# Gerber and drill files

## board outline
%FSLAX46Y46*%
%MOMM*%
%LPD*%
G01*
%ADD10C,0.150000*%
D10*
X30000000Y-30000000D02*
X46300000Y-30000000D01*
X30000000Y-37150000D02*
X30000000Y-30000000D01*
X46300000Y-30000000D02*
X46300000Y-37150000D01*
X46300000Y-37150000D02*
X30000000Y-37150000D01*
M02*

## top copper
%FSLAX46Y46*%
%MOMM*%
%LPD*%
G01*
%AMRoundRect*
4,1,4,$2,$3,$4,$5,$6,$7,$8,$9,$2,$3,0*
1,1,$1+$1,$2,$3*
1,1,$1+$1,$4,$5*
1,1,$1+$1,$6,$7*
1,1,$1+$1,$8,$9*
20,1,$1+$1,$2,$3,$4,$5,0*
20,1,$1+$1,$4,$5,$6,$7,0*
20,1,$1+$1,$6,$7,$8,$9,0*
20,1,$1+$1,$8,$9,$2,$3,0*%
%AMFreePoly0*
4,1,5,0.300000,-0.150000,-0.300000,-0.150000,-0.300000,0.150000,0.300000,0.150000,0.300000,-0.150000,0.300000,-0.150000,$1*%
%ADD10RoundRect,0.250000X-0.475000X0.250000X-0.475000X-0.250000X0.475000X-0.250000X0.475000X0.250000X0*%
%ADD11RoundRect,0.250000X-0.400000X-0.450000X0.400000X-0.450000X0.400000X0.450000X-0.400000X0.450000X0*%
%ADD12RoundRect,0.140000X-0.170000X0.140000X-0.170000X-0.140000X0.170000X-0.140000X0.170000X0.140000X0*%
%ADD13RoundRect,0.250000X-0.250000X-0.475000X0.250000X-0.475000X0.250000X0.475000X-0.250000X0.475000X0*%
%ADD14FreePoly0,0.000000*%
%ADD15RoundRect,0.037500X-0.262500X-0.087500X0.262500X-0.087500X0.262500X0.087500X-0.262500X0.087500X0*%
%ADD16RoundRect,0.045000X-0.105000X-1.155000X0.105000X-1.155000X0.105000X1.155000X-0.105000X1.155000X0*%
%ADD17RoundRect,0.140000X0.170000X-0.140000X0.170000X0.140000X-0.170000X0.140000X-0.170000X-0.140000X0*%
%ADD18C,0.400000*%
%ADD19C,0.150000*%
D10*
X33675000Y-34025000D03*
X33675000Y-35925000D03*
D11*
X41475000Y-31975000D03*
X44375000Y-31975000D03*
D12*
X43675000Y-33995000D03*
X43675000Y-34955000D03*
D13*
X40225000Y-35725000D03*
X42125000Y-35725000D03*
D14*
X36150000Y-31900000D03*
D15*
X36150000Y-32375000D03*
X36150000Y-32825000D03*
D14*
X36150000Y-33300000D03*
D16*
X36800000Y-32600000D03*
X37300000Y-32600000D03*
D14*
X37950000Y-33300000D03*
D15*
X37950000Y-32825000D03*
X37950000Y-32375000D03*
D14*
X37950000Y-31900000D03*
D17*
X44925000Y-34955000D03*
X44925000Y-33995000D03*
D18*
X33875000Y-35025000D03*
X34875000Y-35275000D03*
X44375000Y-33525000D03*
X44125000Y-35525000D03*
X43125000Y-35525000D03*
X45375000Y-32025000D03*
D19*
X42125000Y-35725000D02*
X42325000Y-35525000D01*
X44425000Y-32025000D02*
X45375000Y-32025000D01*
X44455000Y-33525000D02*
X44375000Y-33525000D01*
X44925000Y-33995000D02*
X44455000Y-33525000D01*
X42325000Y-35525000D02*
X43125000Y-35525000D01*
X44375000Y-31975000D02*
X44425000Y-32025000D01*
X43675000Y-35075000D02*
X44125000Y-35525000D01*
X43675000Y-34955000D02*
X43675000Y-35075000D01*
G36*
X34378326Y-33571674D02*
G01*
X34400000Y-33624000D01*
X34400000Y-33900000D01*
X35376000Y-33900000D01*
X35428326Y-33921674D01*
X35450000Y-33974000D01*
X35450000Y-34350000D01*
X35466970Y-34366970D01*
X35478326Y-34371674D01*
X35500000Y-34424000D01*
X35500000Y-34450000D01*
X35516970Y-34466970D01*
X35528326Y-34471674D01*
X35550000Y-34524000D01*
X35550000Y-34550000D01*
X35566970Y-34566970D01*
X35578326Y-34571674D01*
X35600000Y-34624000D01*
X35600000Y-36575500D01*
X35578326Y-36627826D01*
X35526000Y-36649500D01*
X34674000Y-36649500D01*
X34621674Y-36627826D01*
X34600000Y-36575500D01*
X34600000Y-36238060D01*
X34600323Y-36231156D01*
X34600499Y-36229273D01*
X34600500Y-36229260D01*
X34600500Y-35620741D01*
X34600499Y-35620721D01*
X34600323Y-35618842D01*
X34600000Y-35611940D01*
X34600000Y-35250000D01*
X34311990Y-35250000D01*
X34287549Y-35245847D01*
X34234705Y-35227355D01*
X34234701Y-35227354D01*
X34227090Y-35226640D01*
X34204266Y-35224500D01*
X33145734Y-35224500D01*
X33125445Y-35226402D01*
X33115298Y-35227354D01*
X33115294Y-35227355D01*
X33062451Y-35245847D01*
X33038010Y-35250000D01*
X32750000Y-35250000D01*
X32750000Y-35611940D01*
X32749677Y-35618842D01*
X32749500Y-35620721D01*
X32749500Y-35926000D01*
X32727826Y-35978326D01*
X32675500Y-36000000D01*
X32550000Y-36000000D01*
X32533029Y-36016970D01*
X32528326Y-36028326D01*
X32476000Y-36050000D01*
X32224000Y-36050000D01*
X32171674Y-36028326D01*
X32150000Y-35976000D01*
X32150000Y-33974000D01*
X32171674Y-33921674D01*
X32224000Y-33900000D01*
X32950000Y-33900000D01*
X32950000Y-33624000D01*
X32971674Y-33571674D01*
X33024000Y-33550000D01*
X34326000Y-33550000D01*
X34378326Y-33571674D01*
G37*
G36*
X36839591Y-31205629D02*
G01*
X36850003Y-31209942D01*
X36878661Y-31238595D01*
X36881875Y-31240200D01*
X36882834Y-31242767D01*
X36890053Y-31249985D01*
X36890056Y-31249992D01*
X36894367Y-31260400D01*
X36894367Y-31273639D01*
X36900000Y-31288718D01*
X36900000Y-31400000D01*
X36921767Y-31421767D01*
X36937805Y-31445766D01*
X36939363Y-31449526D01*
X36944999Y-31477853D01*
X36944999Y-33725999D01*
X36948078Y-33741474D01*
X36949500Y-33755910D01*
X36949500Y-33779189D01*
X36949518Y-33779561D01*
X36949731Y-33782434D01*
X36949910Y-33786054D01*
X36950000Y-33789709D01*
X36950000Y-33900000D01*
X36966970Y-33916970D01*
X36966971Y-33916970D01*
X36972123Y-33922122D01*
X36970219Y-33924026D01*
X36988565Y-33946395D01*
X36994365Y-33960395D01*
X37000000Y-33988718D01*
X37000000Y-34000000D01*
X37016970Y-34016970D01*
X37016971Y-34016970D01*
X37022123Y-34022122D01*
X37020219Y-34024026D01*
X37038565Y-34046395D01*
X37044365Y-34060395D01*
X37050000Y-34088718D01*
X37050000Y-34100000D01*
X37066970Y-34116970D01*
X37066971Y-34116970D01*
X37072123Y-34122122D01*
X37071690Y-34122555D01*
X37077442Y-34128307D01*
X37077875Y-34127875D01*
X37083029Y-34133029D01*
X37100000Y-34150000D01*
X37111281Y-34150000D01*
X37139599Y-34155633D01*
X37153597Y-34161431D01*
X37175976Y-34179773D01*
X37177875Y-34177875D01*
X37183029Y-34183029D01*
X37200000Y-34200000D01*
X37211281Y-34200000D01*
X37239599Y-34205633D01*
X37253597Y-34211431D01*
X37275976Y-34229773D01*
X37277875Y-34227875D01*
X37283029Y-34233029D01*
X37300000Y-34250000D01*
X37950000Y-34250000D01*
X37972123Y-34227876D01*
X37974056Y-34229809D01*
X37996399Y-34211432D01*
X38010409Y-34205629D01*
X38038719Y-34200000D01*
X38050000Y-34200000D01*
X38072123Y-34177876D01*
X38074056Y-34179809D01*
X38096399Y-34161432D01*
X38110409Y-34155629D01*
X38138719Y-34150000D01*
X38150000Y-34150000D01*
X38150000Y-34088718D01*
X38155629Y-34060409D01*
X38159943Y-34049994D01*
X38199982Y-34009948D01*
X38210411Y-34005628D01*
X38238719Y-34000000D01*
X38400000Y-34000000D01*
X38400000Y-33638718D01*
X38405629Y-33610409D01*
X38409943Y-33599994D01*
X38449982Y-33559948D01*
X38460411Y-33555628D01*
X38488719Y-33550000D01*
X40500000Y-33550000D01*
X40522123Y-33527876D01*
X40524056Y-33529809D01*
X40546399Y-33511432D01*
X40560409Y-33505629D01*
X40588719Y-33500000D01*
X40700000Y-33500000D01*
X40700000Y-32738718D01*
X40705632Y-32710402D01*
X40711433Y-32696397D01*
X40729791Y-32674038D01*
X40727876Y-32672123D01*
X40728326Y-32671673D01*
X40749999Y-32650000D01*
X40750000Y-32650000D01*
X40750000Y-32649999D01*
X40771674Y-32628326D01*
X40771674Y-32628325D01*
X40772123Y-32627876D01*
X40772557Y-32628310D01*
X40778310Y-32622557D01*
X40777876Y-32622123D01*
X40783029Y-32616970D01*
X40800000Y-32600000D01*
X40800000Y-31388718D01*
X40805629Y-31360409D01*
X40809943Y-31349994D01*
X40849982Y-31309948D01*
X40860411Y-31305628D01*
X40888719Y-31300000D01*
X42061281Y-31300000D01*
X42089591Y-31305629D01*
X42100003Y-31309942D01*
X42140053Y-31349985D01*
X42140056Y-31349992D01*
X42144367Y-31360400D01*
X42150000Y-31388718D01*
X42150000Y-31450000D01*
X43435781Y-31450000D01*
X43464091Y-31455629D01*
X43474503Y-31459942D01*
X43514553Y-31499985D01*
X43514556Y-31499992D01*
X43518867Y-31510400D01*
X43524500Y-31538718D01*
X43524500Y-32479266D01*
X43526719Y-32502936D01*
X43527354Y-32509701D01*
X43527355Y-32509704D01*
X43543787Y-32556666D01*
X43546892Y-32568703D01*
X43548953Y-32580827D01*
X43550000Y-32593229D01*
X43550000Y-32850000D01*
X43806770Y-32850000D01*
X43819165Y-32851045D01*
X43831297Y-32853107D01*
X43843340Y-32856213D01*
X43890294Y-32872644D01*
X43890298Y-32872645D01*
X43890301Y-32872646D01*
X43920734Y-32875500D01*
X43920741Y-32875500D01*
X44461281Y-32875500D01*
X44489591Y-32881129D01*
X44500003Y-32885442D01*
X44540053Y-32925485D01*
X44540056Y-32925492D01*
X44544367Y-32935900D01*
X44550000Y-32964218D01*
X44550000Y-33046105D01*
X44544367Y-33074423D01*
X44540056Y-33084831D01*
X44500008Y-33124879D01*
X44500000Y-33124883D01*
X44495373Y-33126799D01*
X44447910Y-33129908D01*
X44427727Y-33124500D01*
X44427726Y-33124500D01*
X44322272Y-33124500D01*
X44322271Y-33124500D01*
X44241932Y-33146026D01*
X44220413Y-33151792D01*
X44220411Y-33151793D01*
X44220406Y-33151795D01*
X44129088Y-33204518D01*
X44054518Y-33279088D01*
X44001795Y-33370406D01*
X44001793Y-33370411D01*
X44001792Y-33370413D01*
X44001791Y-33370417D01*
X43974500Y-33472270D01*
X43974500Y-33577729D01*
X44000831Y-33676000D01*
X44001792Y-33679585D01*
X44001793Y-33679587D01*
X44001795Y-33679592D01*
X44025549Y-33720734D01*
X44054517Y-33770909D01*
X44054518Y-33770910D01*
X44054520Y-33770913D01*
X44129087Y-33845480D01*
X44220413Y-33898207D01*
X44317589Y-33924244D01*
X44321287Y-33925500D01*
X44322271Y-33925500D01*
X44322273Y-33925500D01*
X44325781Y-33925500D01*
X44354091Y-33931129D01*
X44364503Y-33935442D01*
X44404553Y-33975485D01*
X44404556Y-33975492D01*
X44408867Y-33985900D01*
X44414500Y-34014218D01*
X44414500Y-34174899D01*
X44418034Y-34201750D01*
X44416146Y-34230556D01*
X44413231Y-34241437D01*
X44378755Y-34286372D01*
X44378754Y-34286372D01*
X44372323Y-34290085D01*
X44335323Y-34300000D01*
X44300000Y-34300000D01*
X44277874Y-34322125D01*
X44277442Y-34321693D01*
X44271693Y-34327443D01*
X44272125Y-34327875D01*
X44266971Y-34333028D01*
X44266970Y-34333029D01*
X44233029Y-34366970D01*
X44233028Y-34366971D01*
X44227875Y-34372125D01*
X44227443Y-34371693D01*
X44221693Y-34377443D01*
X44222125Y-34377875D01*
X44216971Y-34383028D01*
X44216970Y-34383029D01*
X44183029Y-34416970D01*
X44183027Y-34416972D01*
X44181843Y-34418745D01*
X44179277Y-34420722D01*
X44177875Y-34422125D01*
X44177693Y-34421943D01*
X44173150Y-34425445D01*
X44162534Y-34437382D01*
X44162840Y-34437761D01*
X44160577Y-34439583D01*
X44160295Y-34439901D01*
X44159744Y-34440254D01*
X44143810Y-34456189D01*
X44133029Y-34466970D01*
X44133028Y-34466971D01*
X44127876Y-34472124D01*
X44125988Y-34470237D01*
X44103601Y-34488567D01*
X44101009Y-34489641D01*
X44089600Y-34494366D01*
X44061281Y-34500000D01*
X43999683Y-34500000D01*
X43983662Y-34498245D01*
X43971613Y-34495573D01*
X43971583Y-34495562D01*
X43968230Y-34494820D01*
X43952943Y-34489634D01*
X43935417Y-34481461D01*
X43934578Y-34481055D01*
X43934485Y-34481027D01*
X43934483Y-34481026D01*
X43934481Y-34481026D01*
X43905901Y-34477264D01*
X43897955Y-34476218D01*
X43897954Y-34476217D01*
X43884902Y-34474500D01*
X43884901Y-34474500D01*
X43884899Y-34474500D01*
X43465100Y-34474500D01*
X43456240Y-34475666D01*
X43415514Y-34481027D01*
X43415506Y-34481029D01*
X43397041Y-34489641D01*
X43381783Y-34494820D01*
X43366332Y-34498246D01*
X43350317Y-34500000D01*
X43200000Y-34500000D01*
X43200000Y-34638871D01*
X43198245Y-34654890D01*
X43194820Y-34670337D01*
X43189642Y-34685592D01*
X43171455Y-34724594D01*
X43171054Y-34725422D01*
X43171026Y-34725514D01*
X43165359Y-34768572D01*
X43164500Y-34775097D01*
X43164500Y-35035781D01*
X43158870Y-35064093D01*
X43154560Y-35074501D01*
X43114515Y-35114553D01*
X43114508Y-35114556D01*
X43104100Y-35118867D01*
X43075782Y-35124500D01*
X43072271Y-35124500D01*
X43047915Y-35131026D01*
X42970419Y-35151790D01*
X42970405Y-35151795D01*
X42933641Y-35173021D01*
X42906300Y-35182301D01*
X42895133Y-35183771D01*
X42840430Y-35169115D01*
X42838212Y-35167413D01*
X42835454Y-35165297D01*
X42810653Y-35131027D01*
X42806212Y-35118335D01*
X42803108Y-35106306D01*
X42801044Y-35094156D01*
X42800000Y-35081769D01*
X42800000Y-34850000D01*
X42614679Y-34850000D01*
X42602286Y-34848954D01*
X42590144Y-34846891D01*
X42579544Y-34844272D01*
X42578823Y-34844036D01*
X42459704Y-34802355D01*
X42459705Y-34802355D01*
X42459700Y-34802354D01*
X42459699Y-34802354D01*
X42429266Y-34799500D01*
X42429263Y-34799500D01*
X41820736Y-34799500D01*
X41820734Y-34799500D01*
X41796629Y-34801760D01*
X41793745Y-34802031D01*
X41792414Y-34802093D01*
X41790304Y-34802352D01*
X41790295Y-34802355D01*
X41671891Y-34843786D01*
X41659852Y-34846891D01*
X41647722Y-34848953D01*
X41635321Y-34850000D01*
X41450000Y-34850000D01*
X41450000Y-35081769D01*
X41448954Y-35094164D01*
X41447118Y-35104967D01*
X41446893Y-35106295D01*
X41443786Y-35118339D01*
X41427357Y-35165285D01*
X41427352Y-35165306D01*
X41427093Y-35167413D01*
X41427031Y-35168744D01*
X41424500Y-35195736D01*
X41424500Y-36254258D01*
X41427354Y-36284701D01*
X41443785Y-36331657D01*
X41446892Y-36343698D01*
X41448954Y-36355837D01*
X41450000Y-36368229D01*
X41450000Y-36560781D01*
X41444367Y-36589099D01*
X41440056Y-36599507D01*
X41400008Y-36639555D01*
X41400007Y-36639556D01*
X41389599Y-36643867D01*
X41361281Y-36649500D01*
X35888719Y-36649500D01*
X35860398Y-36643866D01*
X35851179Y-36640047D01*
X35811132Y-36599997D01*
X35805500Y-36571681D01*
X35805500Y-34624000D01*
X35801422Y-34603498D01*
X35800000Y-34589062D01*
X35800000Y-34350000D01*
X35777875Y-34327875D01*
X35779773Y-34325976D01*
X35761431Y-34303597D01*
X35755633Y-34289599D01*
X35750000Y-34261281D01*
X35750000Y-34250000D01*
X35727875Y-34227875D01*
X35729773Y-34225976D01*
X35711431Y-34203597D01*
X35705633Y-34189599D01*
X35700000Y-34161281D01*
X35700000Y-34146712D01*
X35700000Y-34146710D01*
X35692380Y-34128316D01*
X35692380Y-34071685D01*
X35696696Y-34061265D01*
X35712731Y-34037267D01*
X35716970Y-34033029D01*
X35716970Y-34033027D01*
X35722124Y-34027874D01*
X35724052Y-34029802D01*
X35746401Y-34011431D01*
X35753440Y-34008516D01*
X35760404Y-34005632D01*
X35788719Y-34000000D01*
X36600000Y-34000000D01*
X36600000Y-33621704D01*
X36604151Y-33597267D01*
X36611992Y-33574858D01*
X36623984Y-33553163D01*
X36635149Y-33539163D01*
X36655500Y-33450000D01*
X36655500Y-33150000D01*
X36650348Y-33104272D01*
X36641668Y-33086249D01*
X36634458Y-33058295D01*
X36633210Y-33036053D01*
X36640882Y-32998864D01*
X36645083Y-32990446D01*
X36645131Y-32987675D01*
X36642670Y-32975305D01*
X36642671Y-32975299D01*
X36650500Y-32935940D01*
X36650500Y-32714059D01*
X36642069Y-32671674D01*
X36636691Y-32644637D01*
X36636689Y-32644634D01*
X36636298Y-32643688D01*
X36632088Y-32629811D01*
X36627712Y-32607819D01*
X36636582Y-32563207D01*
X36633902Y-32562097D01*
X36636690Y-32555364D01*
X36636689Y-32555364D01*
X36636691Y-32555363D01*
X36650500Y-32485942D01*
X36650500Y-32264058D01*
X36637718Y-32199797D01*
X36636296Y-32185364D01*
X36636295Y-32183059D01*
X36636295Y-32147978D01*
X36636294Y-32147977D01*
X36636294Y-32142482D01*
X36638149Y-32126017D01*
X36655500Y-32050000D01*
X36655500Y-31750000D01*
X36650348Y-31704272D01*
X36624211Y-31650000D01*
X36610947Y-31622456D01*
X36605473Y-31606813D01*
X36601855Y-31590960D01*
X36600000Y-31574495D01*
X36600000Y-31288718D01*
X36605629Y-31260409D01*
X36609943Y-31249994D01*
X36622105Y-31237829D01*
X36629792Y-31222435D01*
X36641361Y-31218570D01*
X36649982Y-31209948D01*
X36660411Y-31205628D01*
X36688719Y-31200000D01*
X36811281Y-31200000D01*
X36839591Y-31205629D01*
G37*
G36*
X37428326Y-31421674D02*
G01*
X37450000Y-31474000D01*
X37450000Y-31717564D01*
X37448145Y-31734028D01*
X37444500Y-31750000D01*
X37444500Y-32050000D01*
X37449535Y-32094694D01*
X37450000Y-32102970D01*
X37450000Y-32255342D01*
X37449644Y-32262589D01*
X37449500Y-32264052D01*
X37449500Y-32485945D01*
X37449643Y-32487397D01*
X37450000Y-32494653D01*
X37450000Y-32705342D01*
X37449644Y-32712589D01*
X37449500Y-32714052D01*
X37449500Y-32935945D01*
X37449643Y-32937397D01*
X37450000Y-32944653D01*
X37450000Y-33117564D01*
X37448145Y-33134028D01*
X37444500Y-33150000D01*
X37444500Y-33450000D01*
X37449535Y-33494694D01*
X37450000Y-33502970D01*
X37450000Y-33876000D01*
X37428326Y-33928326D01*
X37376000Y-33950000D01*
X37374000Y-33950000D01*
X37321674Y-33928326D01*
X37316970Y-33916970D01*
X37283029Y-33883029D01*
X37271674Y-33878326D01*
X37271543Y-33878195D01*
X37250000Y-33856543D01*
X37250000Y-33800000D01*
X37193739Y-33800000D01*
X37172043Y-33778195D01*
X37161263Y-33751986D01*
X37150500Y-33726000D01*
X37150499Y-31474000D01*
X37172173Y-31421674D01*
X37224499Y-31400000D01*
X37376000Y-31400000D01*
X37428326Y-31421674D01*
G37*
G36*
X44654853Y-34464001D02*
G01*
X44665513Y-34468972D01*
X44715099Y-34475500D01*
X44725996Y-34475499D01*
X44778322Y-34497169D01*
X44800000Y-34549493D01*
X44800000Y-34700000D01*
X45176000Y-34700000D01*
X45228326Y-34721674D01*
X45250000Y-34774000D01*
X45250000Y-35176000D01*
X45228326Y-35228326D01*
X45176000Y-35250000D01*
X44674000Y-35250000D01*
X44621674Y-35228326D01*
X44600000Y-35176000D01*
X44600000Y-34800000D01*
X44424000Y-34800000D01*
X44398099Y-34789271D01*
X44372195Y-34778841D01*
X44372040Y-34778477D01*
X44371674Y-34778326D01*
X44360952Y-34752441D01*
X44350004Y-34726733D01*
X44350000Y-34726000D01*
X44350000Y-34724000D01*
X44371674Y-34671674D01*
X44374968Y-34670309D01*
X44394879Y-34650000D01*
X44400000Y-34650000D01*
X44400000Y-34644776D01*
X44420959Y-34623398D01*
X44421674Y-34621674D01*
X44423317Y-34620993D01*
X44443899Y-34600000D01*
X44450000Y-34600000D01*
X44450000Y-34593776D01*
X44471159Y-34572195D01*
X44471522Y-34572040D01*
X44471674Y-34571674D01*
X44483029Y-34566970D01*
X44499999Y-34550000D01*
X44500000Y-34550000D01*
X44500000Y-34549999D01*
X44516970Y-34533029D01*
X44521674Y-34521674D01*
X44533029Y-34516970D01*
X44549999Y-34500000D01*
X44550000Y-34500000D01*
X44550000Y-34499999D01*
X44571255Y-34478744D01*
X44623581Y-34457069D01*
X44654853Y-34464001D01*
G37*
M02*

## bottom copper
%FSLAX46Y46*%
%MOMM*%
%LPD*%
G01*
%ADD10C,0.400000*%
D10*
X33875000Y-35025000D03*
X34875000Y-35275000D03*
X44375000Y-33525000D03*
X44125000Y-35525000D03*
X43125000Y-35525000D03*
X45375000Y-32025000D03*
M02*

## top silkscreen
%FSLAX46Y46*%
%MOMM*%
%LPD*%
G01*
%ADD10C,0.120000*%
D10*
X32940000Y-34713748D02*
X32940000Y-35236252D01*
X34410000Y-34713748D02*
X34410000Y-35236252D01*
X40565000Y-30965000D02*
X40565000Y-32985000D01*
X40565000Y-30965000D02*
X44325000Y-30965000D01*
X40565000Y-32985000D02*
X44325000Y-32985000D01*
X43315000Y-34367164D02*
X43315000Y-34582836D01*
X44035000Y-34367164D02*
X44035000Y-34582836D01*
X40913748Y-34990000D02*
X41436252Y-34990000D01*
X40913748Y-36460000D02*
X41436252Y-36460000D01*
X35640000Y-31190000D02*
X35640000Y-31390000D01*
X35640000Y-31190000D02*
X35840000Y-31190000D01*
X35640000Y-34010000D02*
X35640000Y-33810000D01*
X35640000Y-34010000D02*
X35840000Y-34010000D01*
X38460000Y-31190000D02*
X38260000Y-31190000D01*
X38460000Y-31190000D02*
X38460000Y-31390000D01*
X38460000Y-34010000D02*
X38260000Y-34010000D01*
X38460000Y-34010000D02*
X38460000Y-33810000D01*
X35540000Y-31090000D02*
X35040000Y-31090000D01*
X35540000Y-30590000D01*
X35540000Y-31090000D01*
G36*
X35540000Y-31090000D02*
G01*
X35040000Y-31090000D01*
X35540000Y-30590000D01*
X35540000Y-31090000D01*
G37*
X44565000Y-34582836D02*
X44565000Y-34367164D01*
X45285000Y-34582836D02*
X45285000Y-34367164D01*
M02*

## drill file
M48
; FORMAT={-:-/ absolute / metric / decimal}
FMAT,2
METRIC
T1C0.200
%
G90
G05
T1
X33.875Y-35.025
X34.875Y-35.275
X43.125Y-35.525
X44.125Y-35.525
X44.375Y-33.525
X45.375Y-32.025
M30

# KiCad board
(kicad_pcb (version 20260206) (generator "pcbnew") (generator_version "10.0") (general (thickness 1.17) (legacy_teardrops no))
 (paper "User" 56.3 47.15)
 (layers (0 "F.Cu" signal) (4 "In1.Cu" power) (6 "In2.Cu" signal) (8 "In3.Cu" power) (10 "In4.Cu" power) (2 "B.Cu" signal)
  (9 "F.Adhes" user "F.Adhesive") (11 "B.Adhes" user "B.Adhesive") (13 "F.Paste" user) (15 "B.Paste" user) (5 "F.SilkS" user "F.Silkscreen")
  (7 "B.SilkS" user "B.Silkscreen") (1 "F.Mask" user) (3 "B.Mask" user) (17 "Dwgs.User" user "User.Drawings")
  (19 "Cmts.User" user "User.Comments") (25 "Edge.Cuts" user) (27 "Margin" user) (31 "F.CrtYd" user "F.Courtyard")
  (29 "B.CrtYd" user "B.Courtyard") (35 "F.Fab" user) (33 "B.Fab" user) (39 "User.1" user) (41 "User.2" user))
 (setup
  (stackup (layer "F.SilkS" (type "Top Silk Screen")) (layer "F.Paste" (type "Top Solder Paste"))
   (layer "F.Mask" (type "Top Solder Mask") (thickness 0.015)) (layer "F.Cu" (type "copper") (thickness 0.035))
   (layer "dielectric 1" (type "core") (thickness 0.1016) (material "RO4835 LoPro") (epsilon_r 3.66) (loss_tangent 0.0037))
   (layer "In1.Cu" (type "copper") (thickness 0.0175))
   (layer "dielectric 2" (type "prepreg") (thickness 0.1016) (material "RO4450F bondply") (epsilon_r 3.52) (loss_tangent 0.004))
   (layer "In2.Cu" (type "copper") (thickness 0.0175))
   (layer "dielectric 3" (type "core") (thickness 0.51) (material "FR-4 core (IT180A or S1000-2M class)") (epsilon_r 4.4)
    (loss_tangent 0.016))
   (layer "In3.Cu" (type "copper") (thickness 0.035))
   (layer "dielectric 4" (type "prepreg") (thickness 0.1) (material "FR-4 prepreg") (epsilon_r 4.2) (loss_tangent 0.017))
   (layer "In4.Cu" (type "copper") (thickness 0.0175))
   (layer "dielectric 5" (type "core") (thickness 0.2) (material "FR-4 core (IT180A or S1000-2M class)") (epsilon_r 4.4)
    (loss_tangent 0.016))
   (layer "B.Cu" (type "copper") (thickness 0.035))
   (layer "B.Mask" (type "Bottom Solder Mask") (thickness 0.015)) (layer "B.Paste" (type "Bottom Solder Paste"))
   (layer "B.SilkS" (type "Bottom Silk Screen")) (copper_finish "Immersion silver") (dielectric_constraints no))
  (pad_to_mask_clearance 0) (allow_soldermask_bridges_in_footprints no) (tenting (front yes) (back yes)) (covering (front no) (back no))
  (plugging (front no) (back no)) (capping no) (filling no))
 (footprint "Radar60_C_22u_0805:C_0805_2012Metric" (layer "F.Cu") (at 33.675 34.975 -90)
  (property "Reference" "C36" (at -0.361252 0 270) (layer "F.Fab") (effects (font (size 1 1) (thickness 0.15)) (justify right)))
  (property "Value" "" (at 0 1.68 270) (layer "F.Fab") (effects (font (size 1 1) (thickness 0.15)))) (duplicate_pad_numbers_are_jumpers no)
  (fp_line (start -0.261252 0.735) (end 0.261252 0.735) (stroke (width 0.12) (type solid)) (layer "F.SilkS"))
  (fp_line (start -0.261252 -0.735) (end 0.261252 -0.735) (stroke (width 0.12) (type solid)) (layer "F.SilkS"))
  (pad "1" smd roundrect (at -0.95 0 270) (size 1 1.45) (layers "F.Cu" "F.Mask" "F.Paste") (roundrect_rratio 0.25) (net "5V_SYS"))
  (pad "2" smd roundrect (at 0.95 0 270) (size 1 1.45) (layers "F.Cu" "F.Mask" "F.Paste") (roundrect_rratio 0.25) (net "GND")))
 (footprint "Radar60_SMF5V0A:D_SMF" (layer "F.Cu") (at 42.925 31.975)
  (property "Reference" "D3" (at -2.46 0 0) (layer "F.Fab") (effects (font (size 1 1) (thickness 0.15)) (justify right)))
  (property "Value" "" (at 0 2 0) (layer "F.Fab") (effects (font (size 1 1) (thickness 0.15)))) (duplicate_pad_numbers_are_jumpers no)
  (fp_line (start -2.36 -1.01) (end -2.36 1.01) (stroke (width 0.12) (type solid)) (layer "F.SilkS"))
  (fp_line (start -2.36 -1.01) (end 1.4 -1.01) (stroke (width 0.12) (type solid)) (layer "F.SilkS"))
  (fp_line (start -2.36 1.01) (end 1.4 1.01) (stroke (width 0.12) (type solid)) (layer "F.SilkS"))
  (pad "1" smd roundrect (at -1.45 0) (size 1.3 1.4) (layers "F.Cu" "F.Mask" "F.Paste") (roundrect_rratio 0.1923077) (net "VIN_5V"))
  (pad "2" smd roundrect (at 1.45 0) (size 1.3 1.4) (layers "F.Cu" "F.Mask" "F.Paste") (roundrect_rratio 0.1923077) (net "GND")))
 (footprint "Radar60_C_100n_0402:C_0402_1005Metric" (layer "F.Cu") (at 43.675 34.475 -90)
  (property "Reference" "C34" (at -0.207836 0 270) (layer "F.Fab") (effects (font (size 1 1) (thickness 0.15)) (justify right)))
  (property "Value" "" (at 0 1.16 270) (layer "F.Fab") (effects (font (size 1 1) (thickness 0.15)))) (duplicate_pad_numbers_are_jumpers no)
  (fp_line (start -0.107836 0.36) (end 0.107836 0.36) (stroke (width 0.12) (type solid)) (layer "F.SilkS"))
  (fp_line (start -0.107836 -0.36) (end 0.107836 -0.36) (stroke (width 0.12) (type solid)) (layer "F.SilkS"))
  (pad "1" smd roundrect (at -0.48 0 270) (size 0.56 0.62) (layers "F.Cu" "F.Mask" "F.Paste") (roundrect_rratio 0.25) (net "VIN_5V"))
  (pad "2" smd roundrect (at 0.48 0 270) (size 0.56 0.62) (layers "F.Cu" "F.Mask" "F.Paste") (roundrect_rratio 0.25) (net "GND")))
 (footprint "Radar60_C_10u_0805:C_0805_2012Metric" (layer "F.Cu") (at 41.175 35.725)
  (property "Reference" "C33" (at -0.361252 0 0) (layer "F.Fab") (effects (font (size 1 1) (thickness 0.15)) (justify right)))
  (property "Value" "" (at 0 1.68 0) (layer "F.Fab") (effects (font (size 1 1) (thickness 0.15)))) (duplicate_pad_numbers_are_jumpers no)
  (fp_line (start -0.261252 -0.735) (end 0.261252 -0.735) (stroke (width 0.12) (type solid)) (layer "F.SilkS"))
  (fp_line (start -0.261252 0.735) (end 0.261252 0.735) (stroke (width 0.12) (type solid)) (layer "F.SilkS"))
  (pad "1" smd roundrect (at -0.95 0) (size 1 1.45) (layers "F.Cu" "F.Mask" "F.Paste") (roundrect_rratio 0.25) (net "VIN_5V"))
  (pad "2" smd roundrect (at 0.95 0) (size 1 1.45) (layers "F.Cu" "F.Mask" "F.Paste") (roundrect_rratio 0.25) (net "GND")))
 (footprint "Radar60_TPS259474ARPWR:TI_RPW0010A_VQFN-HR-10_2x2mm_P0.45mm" (layer "F.Cu") (at 37.05 32.6)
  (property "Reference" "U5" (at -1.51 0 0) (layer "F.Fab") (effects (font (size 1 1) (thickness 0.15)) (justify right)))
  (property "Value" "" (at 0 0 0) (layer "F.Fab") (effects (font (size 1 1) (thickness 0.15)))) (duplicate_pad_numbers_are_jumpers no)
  (fp_line (start -1.41 -1.41) (end -1.41 -1.21) (stroke (width 0.12) (type solid)) (layer "F.SilkS"))
  (fp_line (start -1.41 -1.41) (end -1.21 -1.41) (stroke (width 0.12) (type solid)) (layer "F.SilkS"))
  (fp_line (start -1.41 1.41) (end -1.41 1.21) (stroke (width 0.12) (type solid)) (layer "F.SilkS"))
  (fp_line (start -1.41 1.41) (end -1.21 1.41) (stroke (width 0.12) (type solid)) (layer "F.SilkS"))
  (fp_line (start 1.41 -1.41) (end 1.21 -1.41) (stroke (width 0.12) (type solid)) (layer "F.SilkS"))
  (fp_line (start 1.41 -1.41) (end 1.41 -1.21) (stroke (width 0.12) (type solid)) (layer "F.SilkS"))
  (fp_line (start 1.41 1.41) (end 1.21 1.41) (stroke (width 0.12) (type solid)) (layer "F.SilkS"))
  (fp_line (start 1.41 1.41) (end 1.41 1.21) (stroke (width 0.12) (type solid)) (layer "F.SilkS"))
  (fp_poly (pts (xy -1.51 -1.51) (xy -2.01 -1.51) (xy -1.51 -2.01)) (stroke (width 0.12) (type solid)) (fill yes) (layer "F.SilkS"))
  (pad "1" smd custom (at -0.9 -0.7) (size 0.6 0.3) (layers "F.Cu" "F.Mask" "F.Paste") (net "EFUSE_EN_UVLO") (solder_mask_margin 0.05)
   (options (clearance outline) (anchor rect)) (primitives))
  (pad "2" smd roundrect (at -0.9 -0.225) (size 0.6 0.25) (layers "F.Cu" "F.Mask" "F.Paste") (roundrect_rratio 0.15) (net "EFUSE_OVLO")
   (solder_mask_margin 0.05))
  (pad "3" smd roundrect (at -0.9 0.225) (size 0.6 0.25) (layers "F.Cu" "F.Mask" "F.Paste") (roundrect_rratio 0.15) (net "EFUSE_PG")
   (solder_mask_margin 0.05))
  (pad "4" smd custom (at -0.9 0.7) (size 0.6 0.3) (layers "F.Cu" "F.Mask" "F.Paste") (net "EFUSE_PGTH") (solder_mask_margin 0.05)
   (options (clearance outline) (anchor rect)) (primitives))
  (pad "5" smd roundrect (at -0.25 0) (size 0.3 2.4) (layers "F.Cu" "F.Mask" "F.Paste") (roundrect_rratio 0.15) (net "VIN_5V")
   (solder_mask_margin 0.05))
  (pad "6" smd roundrect (at 0.25 0) (size 0.3 2.4) (layers "F.Cu" "F.Mask" "F.Paste") (roundrect_rratio 0.15) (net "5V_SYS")
   (solder_mask_margin 0.05))
  (pad "7" smd custom (at 0.9 0.7) (size 0.6 0.3) (layers "F.Cu" "F.Mask" "F.Paste") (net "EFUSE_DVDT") (solder_mask_margin 0.05)
   (options (clearance outline) (anchor rect)) (primitives))
  (pad "8" smd roundrect (at 0.9 0.225) (size 0.6 0.25) (layers "F.Cu" "F.Mask" "F.Paste") (roundrect_rratio 0.15) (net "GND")
   (solder_mask_margin 0.05))
  (pad "9" smd roundrect (at 0.9 -0.225) (size 0.6 0.25) (layers "F.Cu" "F.Mask" "F.Paste") (roundrect_rratio 0.15) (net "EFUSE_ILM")
   (solder_mask_margin 0.05))
  (pad "10" smd custom (at 0.9 -0.7) (size 0.6 0.3) (layers "F.Cu" "F.Mask" "F.Paste") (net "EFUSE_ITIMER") (solder_mask_margin 0.05)
   (options (clearance outline) (anchor rect)) (primitives)))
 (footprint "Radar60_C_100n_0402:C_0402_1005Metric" (layer "F.Cu") (at 44.925 34.475 90)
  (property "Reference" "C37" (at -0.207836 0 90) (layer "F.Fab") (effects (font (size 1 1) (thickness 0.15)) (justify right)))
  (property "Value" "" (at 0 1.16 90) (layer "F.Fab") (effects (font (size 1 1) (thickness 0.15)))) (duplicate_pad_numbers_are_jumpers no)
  (fp_line (start -0.107836 -0.36) (end 0.107836 -0.36) (stroke (width 0.12) (type solid)) (layer "F.SilkS"))
  (fp_line (start -0.107836 0.36) (end 0.107836 0.36) (stroke (width 0.12) (type solid)) (layer "F.SilkS"))
  (pad "1" smd roundrect (at -0.48 0 90) (size 0.56 0.62) (layers "F.Cu" "F.Mask" "F.Paste") (roundrect_rratio 0.25) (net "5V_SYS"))
  (pad "2" smd roundrect (at 0.48 0 90) (size 0.56 0.62) (layers "F.Cu" "F.Mask" "F.Paste") (roundrect_rratio 0.25) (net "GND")))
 (gr_line (start 30 30) (end 46.3 30) (stroke (width 0.15) (type solid)) (layer "Edge.Cuts"))
 (gr_line (start 30 37.15) (end 30 30) (stroke (width 0.15) (type solid)) (layer "Edge.Cuts"))
 (gr_line (start 46.3 30) (end 46.3 37.15) (stroke (width 0.15) (type solid)) (layer "Edge.Cuts"))
 (gr_line (start 46.3 37.15) (end 30 37.15) (stroke (width 0.15) (type solid)) (layer "Edge.Cuts"))
 (via (at 33.875 35.025) (size 0.4) (drill 0.2) (layers "F.Cu" "B.Cu") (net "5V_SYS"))
 (via (at 34.875 35.275) (size 0.4) (drill 0.2) (layers "F.Cu" "B.Cu") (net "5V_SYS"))
 (segment (start 42.125 35.725) (end 42.325 35.525) (width 0.15) (layer "F.Cu") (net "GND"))
 (segment (start 44.425 32.025) (end 45.375 32.025) (width 0.15) (layer "F.Cu") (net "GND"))
 (segment (start 44.455 33.525) (end 44.375 33.525) (width 0.15) (layer "F.Cu") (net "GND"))
 (segment (start 44.925 33.995) (end 44.455 33.525) (width 0.15) (layer "F.Cu") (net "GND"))
 (segment (start 42.325 35.525) (end 43.125 35.525) (width 0.15) (layer "F.Cu") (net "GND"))
 (segment (start 44.375 31.975) (end 44.425 32.025) (width 0.15) (layer "F.Cu") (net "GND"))
 (segment (start 43.675 35.075) (end 44.125 35.525) (width 0.15) (layer "F.Cu") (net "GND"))
 (segment (start 43.675 34.955) (end 43.675 35.075) (width 0.15) (layer "F.Cu") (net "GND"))
 (via (at 44.375 33.525) (size 0.4) (drill 0.2) (layers "F.Cu" "B.Cu") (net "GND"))
 (via (at 44.125 35.525) (size 0.4) (drill 0.2) (layers "F.Cu" "B.Cu") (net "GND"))
 (via (at 43.125 35.525) (size 0.4) (drill 0.2) (layers "F.Cu" "B.Cu") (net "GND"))
 (via (at 45.375 32.025) (size 0.4) (drill 0.2) (layers "F.Cu" "B.Cu") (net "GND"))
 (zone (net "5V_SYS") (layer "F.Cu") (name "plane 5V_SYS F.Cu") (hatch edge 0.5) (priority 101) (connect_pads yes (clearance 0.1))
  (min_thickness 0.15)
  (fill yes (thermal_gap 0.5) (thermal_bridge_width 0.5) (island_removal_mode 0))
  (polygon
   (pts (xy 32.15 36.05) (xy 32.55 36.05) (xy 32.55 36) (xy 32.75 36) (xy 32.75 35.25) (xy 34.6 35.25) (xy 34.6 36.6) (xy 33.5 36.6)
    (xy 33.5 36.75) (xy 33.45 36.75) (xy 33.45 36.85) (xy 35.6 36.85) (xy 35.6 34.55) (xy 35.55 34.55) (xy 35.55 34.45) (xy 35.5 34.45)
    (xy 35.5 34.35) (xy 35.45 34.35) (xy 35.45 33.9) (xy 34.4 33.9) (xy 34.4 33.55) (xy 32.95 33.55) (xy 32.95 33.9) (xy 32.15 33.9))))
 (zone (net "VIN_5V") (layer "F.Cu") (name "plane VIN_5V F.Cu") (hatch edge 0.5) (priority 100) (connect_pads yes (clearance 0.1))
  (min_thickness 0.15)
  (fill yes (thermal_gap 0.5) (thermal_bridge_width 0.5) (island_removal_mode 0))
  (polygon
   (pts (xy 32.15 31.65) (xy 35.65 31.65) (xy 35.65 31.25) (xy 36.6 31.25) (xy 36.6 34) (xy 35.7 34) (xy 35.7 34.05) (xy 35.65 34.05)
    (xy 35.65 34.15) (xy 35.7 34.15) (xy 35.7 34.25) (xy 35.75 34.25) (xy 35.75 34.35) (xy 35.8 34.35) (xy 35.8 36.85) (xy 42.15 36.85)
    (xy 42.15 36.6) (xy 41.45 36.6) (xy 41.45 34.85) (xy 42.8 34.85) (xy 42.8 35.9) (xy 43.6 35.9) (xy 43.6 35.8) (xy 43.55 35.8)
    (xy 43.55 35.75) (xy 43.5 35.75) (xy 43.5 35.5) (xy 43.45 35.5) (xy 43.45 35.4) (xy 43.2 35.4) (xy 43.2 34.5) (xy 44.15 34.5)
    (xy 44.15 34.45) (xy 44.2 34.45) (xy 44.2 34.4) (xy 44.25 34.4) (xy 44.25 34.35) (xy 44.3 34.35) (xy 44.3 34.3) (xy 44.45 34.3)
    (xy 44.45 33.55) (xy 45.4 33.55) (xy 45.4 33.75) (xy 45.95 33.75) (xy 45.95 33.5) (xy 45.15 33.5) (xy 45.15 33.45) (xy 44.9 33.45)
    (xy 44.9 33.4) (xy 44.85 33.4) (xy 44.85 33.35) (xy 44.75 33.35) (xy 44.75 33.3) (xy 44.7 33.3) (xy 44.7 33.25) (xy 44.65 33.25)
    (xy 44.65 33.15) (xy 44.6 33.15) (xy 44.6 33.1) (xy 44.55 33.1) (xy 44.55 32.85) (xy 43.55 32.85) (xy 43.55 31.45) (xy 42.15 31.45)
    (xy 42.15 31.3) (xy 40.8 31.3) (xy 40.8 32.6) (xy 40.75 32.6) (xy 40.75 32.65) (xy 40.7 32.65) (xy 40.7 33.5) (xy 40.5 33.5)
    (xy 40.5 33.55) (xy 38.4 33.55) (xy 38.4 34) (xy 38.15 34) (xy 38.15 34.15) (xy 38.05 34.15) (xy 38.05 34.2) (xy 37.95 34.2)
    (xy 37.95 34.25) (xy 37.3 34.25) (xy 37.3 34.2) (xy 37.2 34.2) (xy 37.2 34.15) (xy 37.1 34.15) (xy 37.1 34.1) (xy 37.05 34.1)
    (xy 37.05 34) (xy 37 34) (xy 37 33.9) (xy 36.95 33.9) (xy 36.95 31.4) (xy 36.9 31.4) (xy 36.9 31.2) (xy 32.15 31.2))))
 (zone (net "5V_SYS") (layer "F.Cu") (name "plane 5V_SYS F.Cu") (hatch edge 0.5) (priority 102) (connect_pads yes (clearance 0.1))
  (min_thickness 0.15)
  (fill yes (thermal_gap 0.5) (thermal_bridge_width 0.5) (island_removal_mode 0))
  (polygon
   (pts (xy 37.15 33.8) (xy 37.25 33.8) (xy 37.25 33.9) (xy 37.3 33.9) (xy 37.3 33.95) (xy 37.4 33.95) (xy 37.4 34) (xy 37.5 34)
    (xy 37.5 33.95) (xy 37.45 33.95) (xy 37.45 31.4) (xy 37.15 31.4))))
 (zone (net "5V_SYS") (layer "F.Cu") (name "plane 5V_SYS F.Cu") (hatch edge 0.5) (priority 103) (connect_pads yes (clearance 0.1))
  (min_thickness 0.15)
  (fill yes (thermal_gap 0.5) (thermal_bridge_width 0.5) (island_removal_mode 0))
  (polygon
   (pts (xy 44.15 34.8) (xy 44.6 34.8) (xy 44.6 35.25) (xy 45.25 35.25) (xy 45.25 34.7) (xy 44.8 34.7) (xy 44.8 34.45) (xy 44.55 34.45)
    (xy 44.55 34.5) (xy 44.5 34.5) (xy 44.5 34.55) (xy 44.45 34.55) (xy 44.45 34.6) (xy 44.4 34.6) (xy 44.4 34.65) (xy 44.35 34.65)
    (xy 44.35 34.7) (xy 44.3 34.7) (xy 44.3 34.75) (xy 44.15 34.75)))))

